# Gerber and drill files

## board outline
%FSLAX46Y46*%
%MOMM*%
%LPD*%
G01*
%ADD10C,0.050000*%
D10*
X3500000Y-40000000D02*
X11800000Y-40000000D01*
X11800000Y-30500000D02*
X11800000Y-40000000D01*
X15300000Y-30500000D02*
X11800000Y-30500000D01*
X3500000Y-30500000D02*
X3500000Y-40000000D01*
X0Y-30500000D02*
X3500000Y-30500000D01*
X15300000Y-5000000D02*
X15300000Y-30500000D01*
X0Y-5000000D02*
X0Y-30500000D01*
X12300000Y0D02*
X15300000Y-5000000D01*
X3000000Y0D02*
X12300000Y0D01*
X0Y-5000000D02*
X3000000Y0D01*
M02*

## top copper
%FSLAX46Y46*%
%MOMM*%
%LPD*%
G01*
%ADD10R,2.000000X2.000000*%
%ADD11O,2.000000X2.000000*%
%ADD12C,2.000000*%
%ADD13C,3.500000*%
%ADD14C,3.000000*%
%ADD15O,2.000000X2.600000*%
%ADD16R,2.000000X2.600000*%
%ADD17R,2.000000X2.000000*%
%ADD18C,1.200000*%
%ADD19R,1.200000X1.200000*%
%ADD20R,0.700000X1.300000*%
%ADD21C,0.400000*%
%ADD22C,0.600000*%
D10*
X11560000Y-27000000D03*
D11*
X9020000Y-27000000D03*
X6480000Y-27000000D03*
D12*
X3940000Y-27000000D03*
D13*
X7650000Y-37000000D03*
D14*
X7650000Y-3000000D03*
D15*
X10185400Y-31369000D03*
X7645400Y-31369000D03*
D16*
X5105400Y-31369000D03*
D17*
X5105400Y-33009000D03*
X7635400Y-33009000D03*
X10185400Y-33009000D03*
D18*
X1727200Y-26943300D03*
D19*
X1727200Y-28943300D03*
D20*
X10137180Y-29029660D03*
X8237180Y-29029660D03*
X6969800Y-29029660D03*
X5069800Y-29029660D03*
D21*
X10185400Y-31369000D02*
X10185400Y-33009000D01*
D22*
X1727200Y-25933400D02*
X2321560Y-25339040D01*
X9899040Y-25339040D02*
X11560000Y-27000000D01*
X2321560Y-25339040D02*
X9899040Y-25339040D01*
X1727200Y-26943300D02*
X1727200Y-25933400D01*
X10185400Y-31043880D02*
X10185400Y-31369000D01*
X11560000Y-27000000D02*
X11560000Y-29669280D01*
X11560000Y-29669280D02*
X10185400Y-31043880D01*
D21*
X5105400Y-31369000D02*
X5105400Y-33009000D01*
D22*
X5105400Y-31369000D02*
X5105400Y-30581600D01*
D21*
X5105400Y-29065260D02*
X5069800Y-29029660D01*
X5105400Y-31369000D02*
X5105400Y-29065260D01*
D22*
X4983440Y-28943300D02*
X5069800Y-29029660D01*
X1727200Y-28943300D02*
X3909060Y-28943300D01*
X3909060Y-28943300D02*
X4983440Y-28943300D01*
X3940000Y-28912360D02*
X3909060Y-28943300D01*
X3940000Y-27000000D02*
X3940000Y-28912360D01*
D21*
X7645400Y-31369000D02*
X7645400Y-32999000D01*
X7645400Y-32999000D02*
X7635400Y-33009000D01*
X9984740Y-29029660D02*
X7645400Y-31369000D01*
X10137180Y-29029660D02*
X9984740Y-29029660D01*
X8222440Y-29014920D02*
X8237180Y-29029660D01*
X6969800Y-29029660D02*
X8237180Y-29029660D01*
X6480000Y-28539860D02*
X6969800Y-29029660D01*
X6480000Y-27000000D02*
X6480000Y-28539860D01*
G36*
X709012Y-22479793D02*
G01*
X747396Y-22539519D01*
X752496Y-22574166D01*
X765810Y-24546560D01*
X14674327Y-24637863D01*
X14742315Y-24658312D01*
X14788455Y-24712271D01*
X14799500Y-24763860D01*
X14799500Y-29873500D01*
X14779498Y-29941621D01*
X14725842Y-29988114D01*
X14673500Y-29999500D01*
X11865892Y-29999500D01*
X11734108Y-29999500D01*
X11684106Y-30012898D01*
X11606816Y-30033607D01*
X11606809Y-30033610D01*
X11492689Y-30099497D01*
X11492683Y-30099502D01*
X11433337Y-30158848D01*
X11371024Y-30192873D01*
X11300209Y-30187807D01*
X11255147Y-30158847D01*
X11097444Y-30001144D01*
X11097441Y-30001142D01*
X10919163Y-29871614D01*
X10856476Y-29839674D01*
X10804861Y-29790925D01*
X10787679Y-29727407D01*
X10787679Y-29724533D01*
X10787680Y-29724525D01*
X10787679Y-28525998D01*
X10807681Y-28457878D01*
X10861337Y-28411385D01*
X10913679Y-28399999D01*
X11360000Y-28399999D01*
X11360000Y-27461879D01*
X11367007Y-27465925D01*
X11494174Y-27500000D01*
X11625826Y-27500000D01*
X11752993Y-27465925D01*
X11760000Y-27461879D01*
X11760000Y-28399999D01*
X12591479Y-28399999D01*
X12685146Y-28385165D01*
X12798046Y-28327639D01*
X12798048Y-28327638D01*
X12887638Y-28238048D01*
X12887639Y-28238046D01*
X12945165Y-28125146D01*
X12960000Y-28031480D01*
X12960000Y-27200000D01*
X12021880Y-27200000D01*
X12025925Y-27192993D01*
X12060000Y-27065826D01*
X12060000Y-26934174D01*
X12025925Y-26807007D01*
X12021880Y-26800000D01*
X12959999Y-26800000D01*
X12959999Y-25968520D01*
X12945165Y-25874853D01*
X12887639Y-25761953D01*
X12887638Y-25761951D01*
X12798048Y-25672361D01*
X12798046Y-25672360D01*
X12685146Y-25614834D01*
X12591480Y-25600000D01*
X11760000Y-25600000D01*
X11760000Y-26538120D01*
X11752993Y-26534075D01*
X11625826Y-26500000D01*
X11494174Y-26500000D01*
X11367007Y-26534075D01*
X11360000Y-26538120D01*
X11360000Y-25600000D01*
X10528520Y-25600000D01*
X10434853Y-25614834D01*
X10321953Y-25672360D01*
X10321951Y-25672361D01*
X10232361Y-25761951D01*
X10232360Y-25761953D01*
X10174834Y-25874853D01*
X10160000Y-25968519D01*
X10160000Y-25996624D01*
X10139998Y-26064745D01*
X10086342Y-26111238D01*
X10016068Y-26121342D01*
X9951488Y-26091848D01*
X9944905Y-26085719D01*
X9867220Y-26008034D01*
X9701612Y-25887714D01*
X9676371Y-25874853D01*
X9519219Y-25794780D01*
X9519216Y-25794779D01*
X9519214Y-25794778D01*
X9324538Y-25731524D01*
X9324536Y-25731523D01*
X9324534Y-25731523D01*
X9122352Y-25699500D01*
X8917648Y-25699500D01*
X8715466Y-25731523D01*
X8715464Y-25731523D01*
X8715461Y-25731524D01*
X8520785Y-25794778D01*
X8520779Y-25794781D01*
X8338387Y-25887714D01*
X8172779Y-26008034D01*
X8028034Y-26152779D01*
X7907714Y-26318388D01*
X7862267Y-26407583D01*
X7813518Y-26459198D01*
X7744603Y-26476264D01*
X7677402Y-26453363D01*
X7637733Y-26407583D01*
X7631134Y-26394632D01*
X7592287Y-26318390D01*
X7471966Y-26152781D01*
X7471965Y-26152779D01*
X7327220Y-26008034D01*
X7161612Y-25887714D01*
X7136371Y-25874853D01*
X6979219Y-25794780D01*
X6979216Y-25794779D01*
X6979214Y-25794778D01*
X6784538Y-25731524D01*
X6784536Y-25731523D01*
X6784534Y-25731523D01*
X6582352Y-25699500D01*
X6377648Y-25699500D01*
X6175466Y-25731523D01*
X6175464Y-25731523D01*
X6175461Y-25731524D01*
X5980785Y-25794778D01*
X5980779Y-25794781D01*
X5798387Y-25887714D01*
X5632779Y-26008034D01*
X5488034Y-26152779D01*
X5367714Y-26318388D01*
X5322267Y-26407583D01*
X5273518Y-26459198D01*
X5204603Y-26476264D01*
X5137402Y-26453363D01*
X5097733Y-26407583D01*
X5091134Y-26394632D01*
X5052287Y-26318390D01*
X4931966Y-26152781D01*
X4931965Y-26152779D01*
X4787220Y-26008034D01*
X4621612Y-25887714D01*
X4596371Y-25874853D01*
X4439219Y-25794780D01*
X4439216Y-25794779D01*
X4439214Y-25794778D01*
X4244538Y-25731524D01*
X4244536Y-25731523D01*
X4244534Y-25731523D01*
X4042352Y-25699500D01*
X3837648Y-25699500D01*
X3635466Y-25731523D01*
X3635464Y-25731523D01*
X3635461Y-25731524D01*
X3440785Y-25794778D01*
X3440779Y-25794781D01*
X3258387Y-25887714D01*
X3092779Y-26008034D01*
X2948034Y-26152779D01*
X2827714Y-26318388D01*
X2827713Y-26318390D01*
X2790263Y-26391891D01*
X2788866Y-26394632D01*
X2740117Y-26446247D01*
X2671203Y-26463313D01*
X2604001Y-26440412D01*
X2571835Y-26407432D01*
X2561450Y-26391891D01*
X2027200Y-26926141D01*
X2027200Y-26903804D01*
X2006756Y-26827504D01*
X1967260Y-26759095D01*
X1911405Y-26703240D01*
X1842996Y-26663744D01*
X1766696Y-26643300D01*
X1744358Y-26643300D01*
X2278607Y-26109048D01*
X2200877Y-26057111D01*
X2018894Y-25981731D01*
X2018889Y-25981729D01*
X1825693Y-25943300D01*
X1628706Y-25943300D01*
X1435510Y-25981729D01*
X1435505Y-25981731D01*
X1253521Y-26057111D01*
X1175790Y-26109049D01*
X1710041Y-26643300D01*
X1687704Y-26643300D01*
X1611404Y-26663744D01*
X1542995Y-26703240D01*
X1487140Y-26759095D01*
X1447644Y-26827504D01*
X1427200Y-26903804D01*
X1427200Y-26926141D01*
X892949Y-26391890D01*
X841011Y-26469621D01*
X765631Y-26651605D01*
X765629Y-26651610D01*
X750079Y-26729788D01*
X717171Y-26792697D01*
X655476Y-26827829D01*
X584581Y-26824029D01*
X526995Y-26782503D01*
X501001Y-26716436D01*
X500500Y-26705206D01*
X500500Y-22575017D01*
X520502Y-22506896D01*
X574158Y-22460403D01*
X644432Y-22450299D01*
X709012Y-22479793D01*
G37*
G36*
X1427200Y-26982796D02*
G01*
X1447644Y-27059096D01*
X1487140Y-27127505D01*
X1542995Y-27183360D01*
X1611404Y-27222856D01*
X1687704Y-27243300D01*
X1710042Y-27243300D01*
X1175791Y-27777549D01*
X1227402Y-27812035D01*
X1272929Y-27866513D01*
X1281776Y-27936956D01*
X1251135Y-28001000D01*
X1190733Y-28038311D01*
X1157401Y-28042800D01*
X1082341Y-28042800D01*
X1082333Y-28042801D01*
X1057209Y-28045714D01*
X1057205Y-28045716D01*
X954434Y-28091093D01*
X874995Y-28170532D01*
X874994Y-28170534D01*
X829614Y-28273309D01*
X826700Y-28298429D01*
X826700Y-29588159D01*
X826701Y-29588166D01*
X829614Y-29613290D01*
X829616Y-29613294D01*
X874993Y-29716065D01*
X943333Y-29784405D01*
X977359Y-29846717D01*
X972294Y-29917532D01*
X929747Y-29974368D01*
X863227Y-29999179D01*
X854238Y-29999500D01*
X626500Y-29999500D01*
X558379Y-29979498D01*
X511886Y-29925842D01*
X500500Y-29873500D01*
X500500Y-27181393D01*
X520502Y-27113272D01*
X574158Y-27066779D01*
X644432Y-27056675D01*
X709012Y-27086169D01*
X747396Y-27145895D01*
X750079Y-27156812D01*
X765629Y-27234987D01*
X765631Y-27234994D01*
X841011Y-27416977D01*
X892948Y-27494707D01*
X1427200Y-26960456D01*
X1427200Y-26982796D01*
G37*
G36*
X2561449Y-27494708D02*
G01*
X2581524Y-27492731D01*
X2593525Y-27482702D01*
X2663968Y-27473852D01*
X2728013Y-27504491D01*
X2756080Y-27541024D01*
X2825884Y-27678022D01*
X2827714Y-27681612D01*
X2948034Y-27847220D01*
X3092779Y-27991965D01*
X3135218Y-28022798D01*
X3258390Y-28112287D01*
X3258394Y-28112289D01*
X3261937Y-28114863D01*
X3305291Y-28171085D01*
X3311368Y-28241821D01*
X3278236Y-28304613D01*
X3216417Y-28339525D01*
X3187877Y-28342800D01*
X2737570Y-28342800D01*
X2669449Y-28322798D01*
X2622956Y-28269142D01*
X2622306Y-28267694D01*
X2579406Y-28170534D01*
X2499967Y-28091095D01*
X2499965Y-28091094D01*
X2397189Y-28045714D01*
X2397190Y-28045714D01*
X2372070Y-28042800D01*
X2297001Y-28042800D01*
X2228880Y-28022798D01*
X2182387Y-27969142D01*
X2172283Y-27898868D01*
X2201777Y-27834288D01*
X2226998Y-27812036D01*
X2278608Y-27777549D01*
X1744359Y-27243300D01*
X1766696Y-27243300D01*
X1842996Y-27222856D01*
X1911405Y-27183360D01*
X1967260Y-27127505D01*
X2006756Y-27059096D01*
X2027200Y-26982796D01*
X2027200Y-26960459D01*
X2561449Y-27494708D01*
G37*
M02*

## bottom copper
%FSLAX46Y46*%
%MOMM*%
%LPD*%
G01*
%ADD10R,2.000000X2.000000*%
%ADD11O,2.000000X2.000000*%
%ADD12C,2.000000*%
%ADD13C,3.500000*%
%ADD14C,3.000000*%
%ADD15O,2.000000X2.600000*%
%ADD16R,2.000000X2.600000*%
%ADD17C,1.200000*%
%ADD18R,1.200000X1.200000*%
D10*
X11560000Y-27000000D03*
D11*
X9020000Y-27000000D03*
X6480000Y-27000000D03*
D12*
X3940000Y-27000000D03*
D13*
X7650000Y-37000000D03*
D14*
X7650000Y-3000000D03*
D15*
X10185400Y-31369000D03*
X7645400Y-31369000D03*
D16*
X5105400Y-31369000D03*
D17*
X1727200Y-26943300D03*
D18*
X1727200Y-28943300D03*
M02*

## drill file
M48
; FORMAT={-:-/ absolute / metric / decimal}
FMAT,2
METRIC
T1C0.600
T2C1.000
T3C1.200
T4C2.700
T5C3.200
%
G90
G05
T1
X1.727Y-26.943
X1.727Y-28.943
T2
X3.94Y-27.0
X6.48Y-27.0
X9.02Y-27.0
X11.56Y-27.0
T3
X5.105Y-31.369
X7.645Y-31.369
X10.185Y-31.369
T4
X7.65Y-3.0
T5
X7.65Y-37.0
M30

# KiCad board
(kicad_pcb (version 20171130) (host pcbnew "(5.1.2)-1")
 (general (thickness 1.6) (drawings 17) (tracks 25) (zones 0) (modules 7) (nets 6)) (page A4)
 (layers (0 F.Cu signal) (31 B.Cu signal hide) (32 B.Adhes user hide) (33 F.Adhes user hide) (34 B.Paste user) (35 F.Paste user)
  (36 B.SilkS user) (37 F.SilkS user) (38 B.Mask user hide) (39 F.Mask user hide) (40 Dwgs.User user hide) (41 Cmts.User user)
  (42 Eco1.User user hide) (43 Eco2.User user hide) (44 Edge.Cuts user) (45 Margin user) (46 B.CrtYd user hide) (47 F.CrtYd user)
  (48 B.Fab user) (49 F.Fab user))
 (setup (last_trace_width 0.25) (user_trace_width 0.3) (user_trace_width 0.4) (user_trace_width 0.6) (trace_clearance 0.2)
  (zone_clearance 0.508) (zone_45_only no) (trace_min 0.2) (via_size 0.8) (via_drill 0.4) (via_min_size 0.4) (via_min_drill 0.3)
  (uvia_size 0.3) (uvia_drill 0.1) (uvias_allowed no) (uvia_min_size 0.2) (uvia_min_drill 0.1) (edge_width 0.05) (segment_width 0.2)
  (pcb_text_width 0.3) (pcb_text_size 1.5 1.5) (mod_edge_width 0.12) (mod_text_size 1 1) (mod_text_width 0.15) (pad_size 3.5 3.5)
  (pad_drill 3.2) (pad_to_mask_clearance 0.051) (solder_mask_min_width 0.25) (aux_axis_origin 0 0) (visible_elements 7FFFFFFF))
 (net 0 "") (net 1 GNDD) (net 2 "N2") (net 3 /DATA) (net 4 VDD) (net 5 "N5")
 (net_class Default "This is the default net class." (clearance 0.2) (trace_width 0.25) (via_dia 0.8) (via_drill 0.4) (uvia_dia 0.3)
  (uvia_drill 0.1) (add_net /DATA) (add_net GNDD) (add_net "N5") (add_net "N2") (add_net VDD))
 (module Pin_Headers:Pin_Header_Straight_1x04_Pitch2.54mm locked (layer F.Cu) (at 3.94 27 90)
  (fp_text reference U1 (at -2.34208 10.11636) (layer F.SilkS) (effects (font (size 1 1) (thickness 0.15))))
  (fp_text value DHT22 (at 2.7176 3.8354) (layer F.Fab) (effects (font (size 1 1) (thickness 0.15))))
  (pad 4 thru_hole rect (at 0 7.62 90) (size 2 2) (drill 1) (layers *.Cu *.Mask) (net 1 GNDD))
  (pad 3 thru_hole oval (at 0 5.08 90) (size 2 2) (drill 1) (layers *.Cu *.Mask) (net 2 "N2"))
  (pad 2 thru_hole oval (at 0 2.54 90) (size 2 2) (drill 1) (layers *.Cu *.Mask) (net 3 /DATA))
  (pad 1 thru_hole circle (at 0 0 90) (size 2 2) (drill 1) (layers *.Cu *.Mask) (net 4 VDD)))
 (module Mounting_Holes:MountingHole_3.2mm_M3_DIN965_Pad (layer F.Cu) (at 7.65 37)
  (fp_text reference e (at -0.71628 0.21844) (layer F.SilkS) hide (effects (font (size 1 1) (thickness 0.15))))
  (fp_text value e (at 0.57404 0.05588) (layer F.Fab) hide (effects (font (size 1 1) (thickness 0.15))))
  (pad 1 thru_hole circle (at 0 0) (size 3.5 3.5) (drill 3.2) (layers *.Cu *.Mask)))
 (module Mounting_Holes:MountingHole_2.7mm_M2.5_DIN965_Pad (layer F.Cu) (at 7.65 3)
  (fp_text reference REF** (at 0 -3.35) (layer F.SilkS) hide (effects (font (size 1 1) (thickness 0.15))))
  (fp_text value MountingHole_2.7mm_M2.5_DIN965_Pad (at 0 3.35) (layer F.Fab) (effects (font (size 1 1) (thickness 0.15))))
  (pad GNDD thru_hole circle (at 0 0) (size 3 3) (drill 2.7) (layers *.Cu *.Mask)))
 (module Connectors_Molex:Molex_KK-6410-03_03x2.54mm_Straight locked (layer F.Cu) (at 5.1054 31.369)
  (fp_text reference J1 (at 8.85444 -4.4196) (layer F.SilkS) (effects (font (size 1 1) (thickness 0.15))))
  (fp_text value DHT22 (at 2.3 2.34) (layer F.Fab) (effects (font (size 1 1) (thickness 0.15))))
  (pad 3 thru_hole oval (at 5.08 0) (size 2 2.6) (drill 1.2) (layers *.Cu *.Mask) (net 1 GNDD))
  (pad 2 thru_hole oval (at 2.54 0) (size 2 2.6) (drill 1.2) (layers *.Cu *.Mask) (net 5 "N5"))
  (pad 1 thru_hole rect (at 0 0) (size 2 2.6) (drill 1.2) (layers *.Cu *.Mask) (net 4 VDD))
  (pad 1 smd rect (at 0 1.64) (size 2 2) (layers F.Cu F.Paste F.Mask) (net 4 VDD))
  (pad 2 smd rect (at 2.53 1.64) (size 2 2) (layers F.Cu F.Paste F.Mask) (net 5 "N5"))
  (pad 3 smd rect (at 5.08 1.64) (size 2 2) (layers F.Cu F.Paste F.Mask) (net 1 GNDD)))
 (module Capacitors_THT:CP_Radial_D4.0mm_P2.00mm (layer F.Cu) (at 1.7272 28.9433 90)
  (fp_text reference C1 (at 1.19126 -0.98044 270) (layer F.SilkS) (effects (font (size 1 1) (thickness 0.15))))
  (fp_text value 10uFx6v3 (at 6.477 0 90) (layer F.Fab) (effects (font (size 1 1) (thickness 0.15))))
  (pad 2 thru_hole circle (at 2 0 90) (size 1.2 1.2) (drill 0.6) (layers *.Cu *.Mask) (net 1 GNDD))
  (pad 1 thru_hole rect (at 0 0 90) (size 1.2 1.2) (drill 0.6) (layers *.Cu *.Mask) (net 4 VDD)))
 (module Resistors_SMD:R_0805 (layer F.Cu) (at 9.18718 29.02966)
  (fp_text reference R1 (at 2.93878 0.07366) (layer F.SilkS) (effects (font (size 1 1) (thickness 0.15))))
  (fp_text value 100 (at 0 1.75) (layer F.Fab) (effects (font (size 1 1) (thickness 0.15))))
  (pad 2 smd rect (at 0.95 0) (size 0.7 1.3) (layers F.Cu F.Paste F.Mask) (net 5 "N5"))
  (pad 1 smd rect (at -0.95 0) (size 0.7 1.3) (layers F.Cu F.Paste F.Mask) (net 3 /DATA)))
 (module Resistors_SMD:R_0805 (layer F.Cu) (at 6.0198 29.02966 180)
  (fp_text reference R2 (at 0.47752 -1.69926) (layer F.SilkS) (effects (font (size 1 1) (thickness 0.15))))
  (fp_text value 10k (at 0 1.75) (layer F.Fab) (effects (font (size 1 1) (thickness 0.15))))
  (pad 1 smd rect (at -0.95 0 180) (size 0.7 1.3) (layers F.Cu F.Paste F.Mask) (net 3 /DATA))
  (pad 2 smd rect (at 0.95 0 180) (size 0.7 1.3) (layers F.Cu F.Paste F.Mask) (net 4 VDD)))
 (gr_line (start 3.5 40) (end 11.8 40) (layer Edge.Cuts) (width 0.05))
 (gr_line (start 11.8 30.5) (end 11.8 40) (layer Edge.Cuts) (width 0.05))
 (gr_line (start 15.3 30.5) (end 11.8 30.5) (layer Edge.Cuts) (width 0.05))
 (gr_line (start 3.5 30.5) (end 3.5 40) (layer Edge.Cuts) (width 0.05))
 (gr_line (start 0 30.5) (end 3.5 30.5) (layer Edge.Cuts) (width 0.05))
 (gr_line (start 15.3 5) (end 15.3 30.5) (layer Edge.Cuts) (width 0.05))
 (gr_line (start 0 5) (end 0 30.5) (layer Edge.Cuts) (width 0.05))
 (gr_line (start 12.3 0) (end 15.3 5) (layer Edge.Cuts) (width 0.05))
 (gr_line (start 3 0) (end 12.3 0) (layer Edge.Cuts) (width 0.05))
 (gr_line (start 0 5) (end 3 0) (layer Edge.Cuts) (width 0.05))
 (segment (start 10.1854 31.369) (end 10.1854 33.009) (width 0.4) (layer F.Cu) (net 1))
 (segment (start 1.7272 25.9334) (end 2.32156 25.33904) (width 0.6) (layer F.Cu) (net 1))
 (segment (start 9.89904 25.33904) (end 11.56 27) (width 0.6) (layer F.Cu) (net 1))
 (segment (start 2.32156 25.33904) (end 9.89904 25.33904) (width 0.6) (layer F.Cu) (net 1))
 (segment (start 1.7272 26.9433) (end 1.7272 25.9334) (width 0.6) (layer F.Cu) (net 1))
 (segment (start 10.1854 31.04388) (end 10.1854 31.369) (width 0.6) (layer F.Cu) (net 1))
 (segment (start 11.56 27) (end 11.56 29.66928) (width 0.6) (layer F.Cu) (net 1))
 (segment (start 11.56 29.66928) (end 10.1854 31.04388) (width 0.6) (layer F.Cu) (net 1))
 (segment (start 5.1054 31.369) (end 5.1054 33.009) (width 0.4) (layer F.Cu) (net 4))
 (segment (start 5.1054 31.369) (end 5.1054 30.5816) (width 0.6) (layer F.Cu) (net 4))
 (segment (start 5.1054 29.06526) (end 5.0698 29.02966) (width 0.4) (layer F.Cu) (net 4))
 (segment (start 5.1054 31.369) (end 5.1054 29.06526) (width 0.4) (layer F.Cu) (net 4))
 (segment (start 4.98344 28.9433) (end 5.0698 29.02966) (width 0.6) (layer F.Cu) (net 4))
 (segment (start 1.7272 28.9433) (end 3.90906 28.9433) (width 0.6) (layer F.Cu) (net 4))
 (segment (start 3.90906 28.9433) (end 4.98344 28.9433) (width 0.6) (layer F.Cu) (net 4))
 (segment (start 3.94 28.91236) (end 3.90906 28.9433) (width 0.6) (layer F.Cu) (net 4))
 (segment (start 3.94 27) (end 3.94 28.91236) (width 0.6) (layer F.Cu) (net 4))
 (segment (start 7.6454 31.369) (end 7.6454 32.999) (width 0.4) (layer F.Cu) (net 5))
 (segment (start 7.6454 32.999) (end 7.6354 33.009) (width 0.4) (layer F.Cu) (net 5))
 (segment (start 9.98474 29.02966) (end 7.6454 31.369) (width 0.4) (layer F.Cu) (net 5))
 (segment (start 10.13718 29.02966) (end 9.98474 29.02966) (width 0.4) (layer F.Cu) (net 5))
 (segment (start 8.22244 29.01492) (end 8.23718 29.02966) (width 0.4) (layer F.Cu) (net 3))
 (segment (start 6.9698 29.02966) (end 8.23718 29.02966) (width 0.4) (layer F.Cu) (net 3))
 (segment (start 6.48 28.53986) (end 6.9698 29.02966) (width 0.4) (layer F.Cu) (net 3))
 (segment (start 6.48 27) (end 6.48 28.53986) (width 0.4) (layer F.Cu) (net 3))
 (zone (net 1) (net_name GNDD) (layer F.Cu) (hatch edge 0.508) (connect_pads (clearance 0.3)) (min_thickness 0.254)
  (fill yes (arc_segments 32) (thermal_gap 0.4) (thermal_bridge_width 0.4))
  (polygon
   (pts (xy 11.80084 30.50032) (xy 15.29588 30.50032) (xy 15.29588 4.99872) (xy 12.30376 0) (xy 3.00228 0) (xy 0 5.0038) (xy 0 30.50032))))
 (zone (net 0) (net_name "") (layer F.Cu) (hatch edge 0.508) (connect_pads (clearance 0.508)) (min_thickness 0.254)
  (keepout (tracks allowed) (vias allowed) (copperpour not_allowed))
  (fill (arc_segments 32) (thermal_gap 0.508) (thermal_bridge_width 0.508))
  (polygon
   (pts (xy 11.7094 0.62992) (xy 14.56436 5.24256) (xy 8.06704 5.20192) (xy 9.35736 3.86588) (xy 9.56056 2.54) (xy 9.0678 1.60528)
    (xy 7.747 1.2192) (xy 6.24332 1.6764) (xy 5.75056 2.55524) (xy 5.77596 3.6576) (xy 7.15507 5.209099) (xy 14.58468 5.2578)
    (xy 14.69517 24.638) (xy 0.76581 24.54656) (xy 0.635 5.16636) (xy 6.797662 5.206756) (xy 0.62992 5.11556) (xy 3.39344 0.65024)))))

